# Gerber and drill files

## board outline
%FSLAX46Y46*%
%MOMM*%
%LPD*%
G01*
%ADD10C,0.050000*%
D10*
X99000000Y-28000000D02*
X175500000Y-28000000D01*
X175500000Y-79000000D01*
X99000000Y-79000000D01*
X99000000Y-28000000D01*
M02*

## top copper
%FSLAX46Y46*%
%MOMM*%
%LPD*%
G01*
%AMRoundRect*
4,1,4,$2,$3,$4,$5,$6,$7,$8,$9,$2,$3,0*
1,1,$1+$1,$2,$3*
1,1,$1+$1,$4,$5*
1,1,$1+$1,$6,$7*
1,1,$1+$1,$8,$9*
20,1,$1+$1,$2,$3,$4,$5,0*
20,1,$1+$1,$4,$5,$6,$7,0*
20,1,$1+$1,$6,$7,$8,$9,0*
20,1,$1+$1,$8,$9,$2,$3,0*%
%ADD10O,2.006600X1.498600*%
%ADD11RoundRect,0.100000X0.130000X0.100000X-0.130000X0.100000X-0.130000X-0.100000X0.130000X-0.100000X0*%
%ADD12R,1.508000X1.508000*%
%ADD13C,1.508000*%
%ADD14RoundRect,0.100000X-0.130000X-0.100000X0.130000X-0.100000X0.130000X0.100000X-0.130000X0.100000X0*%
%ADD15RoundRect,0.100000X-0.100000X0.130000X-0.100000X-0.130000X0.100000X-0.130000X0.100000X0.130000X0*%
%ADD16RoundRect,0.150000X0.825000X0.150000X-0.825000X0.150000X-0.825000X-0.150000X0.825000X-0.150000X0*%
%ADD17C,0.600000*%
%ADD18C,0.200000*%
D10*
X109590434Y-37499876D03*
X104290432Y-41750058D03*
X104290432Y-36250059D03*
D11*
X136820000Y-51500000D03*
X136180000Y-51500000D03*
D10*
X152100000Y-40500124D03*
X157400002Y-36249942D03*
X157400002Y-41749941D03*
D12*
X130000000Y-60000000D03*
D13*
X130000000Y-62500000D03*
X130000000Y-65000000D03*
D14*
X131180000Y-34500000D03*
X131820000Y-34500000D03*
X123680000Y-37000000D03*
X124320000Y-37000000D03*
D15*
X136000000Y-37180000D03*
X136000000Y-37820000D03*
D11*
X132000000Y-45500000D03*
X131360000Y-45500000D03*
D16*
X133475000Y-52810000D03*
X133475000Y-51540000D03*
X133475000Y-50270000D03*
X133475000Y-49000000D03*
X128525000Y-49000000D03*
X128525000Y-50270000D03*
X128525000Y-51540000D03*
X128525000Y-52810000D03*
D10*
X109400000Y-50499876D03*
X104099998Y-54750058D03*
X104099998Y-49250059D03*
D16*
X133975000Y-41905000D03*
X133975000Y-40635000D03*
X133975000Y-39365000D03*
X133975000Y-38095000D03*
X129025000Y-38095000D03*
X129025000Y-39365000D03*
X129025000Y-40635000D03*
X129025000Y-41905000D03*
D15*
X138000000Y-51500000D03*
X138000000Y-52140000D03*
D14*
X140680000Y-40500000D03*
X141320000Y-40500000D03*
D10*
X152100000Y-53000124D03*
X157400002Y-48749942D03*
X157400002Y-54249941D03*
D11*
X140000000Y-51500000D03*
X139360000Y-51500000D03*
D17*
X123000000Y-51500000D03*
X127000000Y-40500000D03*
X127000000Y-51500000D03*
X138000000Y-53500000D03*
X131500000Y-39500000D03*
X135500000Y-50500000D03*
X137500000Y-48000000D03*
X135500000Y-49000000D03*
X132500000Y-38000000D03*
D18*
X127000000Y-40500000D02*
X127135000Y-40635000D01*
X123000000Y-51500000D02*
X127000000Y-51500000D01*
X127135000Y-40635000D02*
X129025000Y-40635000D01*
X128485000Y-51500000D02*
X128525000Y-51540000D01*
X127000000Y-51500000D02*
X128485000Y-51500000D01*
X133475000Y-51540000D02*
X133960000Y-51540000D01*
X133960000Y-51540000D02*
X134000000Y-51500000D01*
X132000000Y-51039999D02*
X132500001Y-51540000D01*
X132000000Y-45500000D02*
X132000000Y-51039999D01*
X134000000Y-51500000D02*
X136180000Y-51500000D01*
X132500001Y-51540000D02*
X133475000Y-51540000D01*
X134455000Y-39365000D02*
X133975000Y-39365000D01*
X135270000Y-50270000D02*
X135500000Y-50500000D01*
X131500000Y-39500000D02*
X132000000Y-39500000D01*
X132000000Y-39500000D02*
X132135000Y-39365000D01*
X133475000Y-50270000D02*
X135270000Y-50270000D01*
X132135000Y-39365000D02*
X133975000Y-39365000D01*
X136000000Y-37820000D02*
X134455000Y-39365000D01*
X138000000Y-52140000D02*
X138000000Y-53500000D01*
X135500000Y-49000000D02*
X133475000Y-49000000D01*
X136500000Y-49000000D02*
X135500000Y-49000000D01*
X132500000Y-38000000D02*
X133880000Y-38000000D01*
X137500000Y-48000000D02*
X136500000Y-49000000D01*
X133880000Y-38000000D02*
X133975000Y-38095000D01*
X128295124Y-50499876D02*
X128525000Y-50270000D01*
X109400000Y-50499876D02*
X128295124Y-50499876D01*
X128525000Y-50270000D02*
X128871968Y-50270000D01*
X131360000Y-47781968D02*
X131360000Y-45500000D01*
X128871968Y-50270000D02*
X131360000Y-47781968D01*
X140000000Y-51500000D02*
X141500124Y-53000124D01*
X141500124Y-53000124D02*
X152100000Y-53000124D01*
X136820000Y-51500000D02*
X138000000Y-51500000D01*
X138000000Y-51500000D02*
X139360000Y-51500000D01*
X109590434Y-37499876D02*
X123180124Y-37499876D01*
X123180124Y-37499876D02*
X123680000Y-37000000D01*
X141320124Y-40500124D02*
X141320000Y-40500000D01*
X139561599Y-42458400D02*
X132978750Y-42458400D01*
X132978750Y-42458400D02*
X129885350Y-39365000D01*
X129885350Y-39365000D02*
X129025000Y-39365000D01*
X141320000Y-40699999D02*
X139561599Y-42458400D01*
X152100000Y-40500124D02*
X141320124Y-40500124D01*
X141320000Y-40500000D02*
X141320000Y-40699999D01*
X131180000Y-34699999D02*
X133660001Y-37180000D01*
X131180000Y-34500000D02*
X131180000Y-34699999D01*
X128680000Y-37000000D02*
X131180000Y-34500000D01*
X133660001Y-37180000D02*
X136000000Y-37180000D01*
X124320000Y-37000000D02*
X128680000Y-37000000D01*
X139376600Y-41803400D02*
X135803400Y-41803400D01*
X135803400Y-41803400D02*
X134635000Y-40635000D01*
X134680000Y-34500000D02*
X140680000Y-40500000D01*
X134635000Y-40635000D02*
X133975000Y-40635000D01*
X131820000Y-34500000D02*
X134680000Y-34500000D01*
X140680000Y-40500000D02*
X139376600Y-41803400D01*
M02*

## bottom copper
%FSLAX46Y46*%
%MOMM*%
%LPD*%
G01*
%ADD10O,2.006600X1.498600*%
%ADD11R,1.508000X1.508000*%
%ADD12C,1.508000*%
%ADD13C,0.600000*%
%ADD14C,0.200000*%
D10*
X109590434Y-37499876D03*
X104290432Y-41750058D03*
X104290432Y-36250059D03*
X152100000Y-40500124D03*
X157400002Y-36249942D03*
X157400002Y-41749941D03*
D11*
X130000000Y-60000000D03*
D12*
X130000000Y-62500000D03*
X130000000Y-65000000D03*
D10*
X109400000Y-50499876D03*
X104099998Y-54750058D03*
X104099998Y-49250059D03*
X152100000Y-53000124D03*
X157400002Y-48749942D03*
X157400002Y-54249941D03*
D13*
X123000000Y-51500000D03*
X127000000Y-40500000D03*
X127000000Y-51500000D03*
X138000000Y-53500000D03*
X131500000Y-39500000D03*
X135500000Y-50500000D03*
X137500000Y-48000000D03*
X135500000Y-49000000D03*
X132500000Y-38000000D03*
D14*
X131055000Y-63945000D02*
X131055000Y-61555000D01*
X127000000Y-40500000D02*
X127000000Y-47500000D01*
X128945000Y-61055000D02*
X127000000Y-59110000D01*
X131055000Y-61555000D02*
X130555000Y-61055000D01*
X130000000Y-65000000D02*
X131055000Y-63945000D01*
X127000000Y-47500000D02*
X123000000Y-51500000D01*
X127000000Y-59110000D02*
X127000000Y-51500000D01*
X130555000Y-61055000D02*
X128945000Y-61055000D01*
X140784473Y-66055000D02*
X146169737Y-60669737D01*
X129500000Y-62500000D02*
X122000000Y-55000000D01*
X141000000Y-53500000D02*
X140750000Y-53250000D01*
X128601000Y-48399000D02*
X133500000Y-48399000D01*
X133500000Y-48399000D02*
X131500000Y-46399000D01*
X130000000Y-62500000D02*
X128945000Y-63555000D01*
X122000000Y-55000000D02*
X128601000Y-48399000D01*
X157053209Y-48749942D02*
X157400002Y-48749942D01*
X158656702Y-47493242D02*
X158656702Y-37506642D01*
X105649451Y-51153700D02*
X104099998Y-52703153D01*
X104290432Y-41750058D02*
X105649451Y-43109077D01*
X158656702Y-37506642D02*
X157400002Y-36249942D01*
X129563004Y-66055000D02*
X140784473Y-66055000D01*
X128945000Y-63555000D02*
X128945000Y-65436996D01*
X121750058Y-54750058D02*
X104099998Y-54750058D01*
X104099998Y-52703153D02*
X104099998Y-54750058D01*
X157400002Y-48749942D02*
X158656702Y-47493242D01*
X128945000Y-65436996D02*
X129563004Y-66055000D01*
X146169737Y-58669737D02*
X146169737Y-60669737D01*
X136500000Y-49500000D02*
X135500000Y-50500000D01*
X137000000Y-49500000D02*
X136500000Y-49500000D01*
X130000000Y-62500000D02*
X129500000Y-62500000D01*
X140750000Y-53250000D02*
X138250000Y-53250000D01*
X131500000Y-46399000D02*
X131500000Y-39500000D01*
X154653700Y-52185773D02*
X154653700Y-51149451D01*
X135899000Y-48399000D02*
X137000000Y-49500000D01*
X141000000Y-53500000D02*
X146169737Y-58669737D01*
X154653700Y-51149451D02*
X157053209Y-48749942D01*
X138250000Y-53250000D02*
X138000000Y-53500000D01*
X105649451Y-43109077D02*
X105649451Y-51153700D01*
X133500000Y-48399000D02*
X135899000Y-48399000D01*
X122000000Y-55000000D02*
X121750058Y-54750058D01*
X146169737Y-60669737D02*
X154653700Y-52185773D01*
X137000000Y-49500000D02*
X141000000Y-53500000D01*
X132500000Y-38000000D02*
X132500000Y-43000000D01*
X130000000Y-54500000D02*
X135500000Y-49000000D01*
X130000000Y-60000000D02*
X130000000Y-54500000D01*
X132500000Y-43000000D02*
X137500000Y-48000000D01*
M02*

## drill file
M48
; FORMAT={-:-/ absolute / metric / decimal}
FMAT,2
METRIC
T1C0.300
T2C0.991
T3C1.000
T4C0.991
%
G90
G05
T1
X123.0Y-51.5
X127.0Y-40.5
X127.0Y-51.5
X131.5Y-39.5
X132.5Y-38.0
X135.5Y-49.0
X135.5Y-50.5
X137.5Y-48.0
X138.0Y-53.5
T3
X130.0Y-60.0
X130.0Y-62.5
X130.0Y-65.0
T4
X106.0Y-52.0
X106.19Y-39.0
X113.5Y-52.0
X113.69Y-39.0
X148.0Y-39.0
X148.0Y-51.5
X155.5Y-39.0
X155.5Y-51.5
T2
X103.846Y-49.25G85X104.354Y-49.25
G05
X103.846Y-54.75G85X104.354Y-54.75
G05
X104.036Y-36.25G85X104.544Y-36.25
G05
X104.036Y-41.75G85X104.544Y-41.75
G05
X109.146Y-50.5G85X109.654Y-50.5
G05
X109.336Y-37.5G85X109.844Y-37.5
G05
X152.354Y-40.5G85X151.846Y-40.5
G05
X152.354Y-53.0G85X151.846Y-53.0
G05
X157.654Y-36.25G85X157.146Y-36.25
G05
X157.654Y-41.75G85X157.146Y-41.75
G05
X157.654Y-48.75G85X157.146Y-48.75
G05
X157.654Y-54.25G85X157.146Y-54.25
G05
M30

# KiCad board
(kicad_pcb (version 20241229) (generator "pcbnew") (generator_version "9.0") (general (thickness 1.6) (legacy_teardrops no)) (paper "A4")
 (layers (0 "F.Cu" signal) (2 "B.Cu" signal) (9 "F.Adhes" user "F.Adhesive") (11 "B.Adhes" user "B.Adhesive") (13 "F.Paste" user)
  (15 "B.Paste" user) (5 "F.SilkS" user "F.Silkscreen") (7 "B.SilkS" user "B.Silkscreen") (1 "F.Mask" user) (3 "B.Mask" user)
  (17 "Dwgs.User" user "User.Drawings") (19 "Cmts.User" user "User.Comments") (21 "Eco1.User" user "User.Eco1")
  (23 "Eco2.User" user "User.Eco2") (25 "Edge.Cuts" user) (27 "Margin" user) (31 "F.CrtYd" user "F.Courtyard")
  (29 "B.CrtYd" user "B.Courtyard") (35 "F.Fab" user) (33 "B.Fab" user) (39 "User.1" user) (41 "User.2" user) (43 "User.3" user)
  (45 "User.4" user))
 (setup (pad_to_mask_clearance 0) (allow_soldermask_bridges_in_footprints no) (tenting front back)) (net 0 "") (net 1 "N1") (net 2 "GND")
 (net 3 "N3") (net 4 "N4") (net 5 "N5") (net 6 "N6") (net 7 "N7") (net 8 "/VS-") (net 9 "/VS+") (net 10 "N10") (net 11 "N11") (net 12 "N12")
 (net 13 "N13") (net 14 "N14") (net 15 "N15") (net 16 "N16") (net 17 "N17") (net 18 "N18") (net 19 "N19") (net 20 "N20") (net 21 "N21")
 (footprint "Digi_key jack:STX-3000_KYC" (layer "F.Cu") (at 109.590434 37.499876 -90)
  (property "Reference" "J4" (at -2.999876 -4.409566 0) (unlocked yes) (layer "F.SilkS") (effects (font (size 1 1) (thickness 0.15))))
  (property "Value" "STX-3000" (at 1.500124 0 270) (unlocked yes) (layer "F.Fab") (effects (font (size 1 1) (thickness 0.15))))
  (pad "" np_thru_hole circle (at 1.500124 -4.1 270) (size 0.9906 0.9906) (drill 0.9906) (layers "*.Cu" "*.Mask"))
  (pad "" np_thru_hole circle (at 1.500124 3.4 270) (size 0.9906 0.9906) (drill 0.9906) (layers "*.Cu" "*.Mask"))
  (pad "1" thru_hole oval (at 0 0) (size 2.0066 1.4986) (drill oval 1.4986 0.9906) (layers "*.Cu" "*.Mask") (remove_unused_layers no)
   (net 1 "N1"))
  (pad "2" thru_hole oval (at 4.250182 5.300002) (size 2.0066 1.4986) (drill oval 1.4986 0.9906) (layers "*.Cu" "*.Mask")
   (remove_unused_layers no) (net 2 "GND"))
  (pad "3" thru_hole oval (at -1.249817 5.300002) (size 2.0066 1.4986) (drill oval 1.4986 0.9906) (layers "*.Cu" "*.Mask")
   (remove_unused_layers no) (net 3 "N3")))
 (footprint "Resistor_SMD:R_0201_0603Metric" (layer "F.Cu") (at 136.5 51.5 180)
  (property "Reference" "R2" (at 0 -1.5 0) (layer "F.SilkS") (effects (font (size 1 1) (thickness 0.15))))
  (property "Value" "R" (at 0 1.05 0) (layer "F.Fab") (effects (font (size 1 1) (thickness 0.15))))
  (pad "" smd roundrect (at -0.345 0 180) (size 0.318 0.36) (layers "F.Paste") (roundrect_rratio 0.25))
  (pad "" smd roundrect (at 0.345 0 180) (size 0.318 0.36) (layers "F.Paste") (roundrect_rratio 0.25))
  (pad "1" smd roundrect (at -0.32 0 180) (size 0.46 0.4) (layers "F.Cu" "F.Mask") (roundrect_rratio 0.25) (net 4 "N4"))
  (pad "2" smd roundrect (at 0.32 0 180) (size 0.46 0.4) (layers "F.Cu" "F.Mask") (roundrect_rratio 0.25) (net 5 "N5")))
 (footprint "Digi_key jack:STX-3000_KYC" (layer "F.Cu") (at 152.1 40.500124 90)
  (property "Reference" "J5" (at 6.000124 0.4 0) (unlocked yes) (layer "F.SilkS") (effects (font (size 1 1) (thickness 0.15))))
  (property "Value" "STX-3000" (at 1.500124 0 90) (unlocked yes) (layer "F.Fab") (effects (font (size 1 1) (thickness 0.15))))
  (pad "" np_thru_hole circle (at 1.500124 -4.1 90) (size 0.9906 0.9906) (drill 0.9906) (layers "*.Cu" "*.Mask"))
  (pad "" np_thru_hole circle (at 1.500124 3.4 90) (size 0.9906 0.9906) (drill 0.9906) (layers "*.Cu" "*.Mask"))
  (pad "1" thru_hole oval (at 0 0 180) (size 2.0066 1.4986) (drill oval 1.4986 0.9906) (layers "*.Cu" "*.Mask") (remove_unused_layers no)
   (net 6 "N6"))
  (pad "2" thru_hole oval (at 4.250182 5.300002 180) (size 2.0066 1.4986) (drill oval 1.4986 0.9906) (layers "*.Cu" "*.Mask")
   (remove_unused_layers no) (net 2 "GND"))
  (pad "3" thru_hole oval (at -1.249817 5.300002 180) (size 2.0066 1.4986) (drill oval 1.4986 0.9906) (layers "*.Cu" "*.Mask")
   (remove_unused_layers no) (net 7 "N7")))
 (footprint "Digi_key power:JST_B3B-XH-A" (layer "F.Cu") (at 129.475 62.5 90)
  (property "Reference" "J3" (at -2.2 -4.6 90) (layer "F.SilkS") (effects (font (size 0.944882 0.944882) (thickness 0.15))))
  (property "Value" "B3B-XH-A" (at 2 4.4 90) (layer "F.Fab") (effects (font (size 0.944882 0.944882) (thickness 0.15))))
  (pad "1" thru_hole rect (at 2.5 0.525 90) (size 1.508 1.508) (drill 1) (layers "*.Cu" "*.Mask") (remove_unused_layers no) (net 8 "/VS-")
   (solder_mask_margin 0.102))
  (pad "2" thru_hole circle (at 0 0.525 90) (size 1.508 1.508) (drill 1) (layers "*.Cu" "*.Mask") (remove_unused_layers no) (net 2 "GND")
   (solder_mask_margin 0.102))
  (pad "3" thru_hole circle (at -2.5 0.525 90) (size 1.508 1.508) (drill 1) (layers "*.Cu" "*.Mask") (remove_unused_layers no)
   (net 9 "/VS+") (solder_mask_margin 0.102)))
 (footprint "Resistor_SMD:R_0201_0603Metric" (layer "F.Cu") (at 131.5 34.5)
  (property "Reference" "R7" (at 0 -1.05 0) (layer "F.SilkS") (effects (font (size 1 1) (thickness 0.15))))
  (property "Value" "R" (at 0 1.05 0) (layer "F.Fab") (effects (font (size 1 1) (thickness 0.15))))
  (pad "" smd roundrect (at -0.345 0) (size 0.318 0.36) (layers "F.Paste") (roundrect_rratio 0.25))
  (pad "" smd roundrect (at 0.345 0) (size 0.318 0.36) (layers "F.Paste") (roundrect_rratio 0.25))
  (pad "1" smd roundrect (at -0.32 0) (size 0.46 0.4) (layers "F.Cu" "F.Mask") (roundrect_rratio 0.25) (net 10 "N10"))
  (pad "2" smd roundrect (at 0.32 0) (size 0.46 0.4) (layers "F.Cu" "F.Mask") (roundrect_rratio 0.25) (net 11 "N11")))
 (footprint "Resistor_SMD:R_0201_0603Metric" (layer "F.Cu") (at 124 37)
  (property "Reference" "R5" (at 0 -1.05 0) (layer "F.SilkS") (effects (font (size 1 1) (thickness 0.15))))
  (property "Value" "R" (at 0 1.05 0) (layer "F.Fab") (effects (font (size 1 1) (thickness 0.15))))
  (pad "" smd roundrect (at -0.345 0) (size 0.318 0.36) (layers "F.Paste") (roundrect_rratio 0.25))
  (pad "" smd roundrect (at 0.345 0) (size 0.318 0.36) (layers "F.Paste") (roundrect_rratio 0.25))
  (pad "1" smd roundrect (at -0.32 0) (size 0.46 0.4) (layers "F.Cu" "F.Mask") (roundrect_rratio 0.25) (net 1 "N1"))
  (pad "2" smd roundrect (at 0.32 0) (size 0.46 0.4) (layers "F.Cu" "F.Mask") (roundrect_rratio 0.25) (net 10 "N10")))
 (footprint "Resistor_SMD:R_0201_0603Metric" (layer "F.Cu") (at 136 37.5 -90)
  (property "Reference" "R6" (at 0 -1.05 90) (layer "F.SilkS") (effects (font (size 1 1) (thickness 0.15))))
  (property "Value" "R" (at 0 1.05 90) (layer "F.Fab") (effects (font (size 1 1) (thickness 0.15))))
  (pad "" smd roundrect (at -0.345 0 270) (size 0.318 0.36) (layers "F.Paste") (roundrect_rratio 0.25))
  (pad "" smd roundrect (at 0.345 0 270) (size 0.318 0.36) (layers "F.Paste") (roundrect_rratio 0.25))
  (pad "1" smd roundrect (at -0.32 0 270) (size 0.46 0.4) (layers "F.Cu" "F.Mask") (roundrect_rratio 0.25) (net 10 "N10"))
  (pad "2" smd roundrect (at 0.32 0 270) (size 0.46 0.4) (layers "F.Cu" "F.Mask") (roundrect_rratio 0.25) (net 2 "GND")))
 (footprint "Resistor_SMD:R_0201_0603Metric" (layer "F.Cu") (at 131.68 45.5 180)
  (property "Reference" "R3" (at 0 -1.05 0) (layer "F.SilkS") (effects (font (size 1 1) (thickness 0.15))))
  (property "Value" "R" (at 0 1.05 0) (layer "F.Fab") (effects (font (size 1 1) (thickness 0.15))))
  (pad "" smd roundrect (at -0.345 0 180) (size 0.318 0.36) (layers "F.Paste") (roundrect_rratio 0.25))
  (pad "" smd roundrect (at 0.345 0 180) (size 0.318 0.36) (layers "F.Paste") (roundrect_rratio 0.25))
  (pad "1" smd roundrect (at -0.32 0 180) (size 0.46 0.4) (layers "F.Cu" "F.Mask") (roundrect_rratio 0.25) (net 5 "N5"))
  (pad "2" smd roundrect (at 0.32 0 180) (size 0.46 0.4) (layers "F.Cu" "F.Mask") (roundrect_rratio 0.25) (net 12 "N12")))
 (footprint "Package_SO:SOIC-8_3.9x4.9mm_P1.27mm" (layer "F.Cu") (at 131 50.905 180)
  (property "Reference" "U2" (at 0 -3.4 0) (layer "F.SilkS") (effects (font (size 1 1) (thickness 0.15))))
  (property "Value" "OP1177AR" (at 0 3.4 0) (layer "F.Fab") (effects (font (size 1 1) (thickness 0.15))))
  (pad "1" smd roundrect (at -2.475 -1.905 180) (size 1.95 0.6) (layers "F.Cu" "F.Mask" "F.Paste") (roundrect_rratio 0.25) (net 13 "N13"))
  (pad "2" smd roundrect (at -2.475 -0.635 180) (size 1.95 0.6) (layers "F.Cu" "F.Mask" "F.Paste") (roundrect_rratio 0.25) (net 5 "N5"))
  (pad "3" smd roundrect (at -2.475 0.635 180) (size 1.95 0.6) (layers "F.Cu" "F.Mask" "F.Paste") (roundrect_rratio 0.25) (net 2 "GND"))
  (pad "4" smd roundrect (at -2.475 1.905 180) (size 1.95 0.6) (layers "F.Cu" "F.Mask" "F.Paste") (roundrect_rratio 0.25) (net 8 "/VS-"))
  (pad "5" smd roundrect (at 2.475 1.905 180) (size 1.95 0.6) (layers "F.Cu" "F.Mask" "F.Paste") (roundrect_rratio 0.25) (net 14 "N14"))
  (pad "6" smd roundrect (at 2.475 0.635 180) (size 1.95 0.6) (layers "F.Cu" "F.Mask" "F.Paste") (roundrect_rratio 0.25) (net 12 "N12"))
  (pad "7" smd roundrect (at 2.475 -0.635 180) (size 1.95 0.6) (layers "F.Cu" "F.Mask" "F.Paste") (roundrect_rratio 0.25) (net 9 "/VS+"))
  (pad "8" smd roundrect (at 2.475 -1.905 180) (size 1.95 0.6) (layers "F.Cu" "F.Mask" "F.Paste") (roundrect_rratio 0.25) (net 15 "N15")))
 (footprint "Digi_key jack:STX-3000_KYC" (layer "F.Cu") (at 109.4 50.499876 -90)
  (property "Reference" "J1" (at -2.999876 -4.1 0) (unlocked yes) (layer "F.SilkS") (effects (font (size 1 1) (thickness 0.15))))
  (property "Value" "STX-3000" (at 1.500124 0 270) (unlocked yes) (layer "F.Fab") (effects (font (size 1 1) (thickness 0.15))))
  (pad "" np_thru_hole circle (at 1.500124 -4.1 270) (size 0.9906 0.9906) (drill 0.9906) (layers "*.Cu" "*.Mask"))
  (pad "" np_thru_hole circle (at 1.500124 3.4 270) (size 0.9906 0.9906) (drill 0.9906) (layers "*.Cu" "*.Mask"))
  (pad "1" thru_hole oval (at 0 0) (size 2.0066 1.4986) (drill oval 1.4986 0.9906) (layers "*.Cu" "*.Mask") (remove_unused_layers no)
   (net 12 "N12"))
  (pad "2" thru_hole oval (at 4.250182 5.300002) (size 2.0066 1.4986) (drill oval 1.4986 0.9906) (layers "*.Cu" "*.Mask")
   (remove_unused_layers no) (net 2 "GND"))
  (pad "3" thru_hole oval (at -1.249817 5.300002) (size 2.0066 1.4986) (drill oval 1.4986 0.9906) (layers "*.Cu" "*.Mask")
   (remove_unused_layers no) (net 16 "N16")))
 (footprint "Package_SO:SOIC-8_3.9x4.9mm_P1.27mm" (layer "F.Cu") (at 131.5 40 180)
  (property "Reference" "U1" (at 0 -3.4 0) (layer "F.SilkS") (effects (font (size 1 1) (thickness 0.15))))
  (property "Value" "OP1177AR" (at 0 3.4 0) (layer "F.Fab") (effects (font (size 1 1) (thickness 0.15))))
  (pad "1" smd roundrect (at -2.475 -1.905 180) (size 1.95 0.6) (layers "F.Cu" "F.Mask" "F.Paste") (roundrect_rratio 0.25) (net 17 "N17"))
  (pad "2" smd roundrect (at -2.475 -0.635 180) (size 1.95 0.6) (layers "F.Cu" "F.Mask" "F.Paste") (roundrect_rratio 0.25) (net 11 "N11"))
  (pad "3" smd roundrect (at -2.475 0.635 180) (size 1.95 0.6) (layers "F.Cu" "F.Mask" "F.Paste") (roundrect_rratio 0.25) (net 2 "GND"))
  (pad "4" smd roundrect (at -2.475 1.905 180) (size 1.95 0.6) (layers "F.Cu" "F.Mask" "F.Paste") (roundrect_rratio 0.25) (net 8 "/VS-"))
  (pad "5" smd roundrect (at 2.475 1.905 180) (size 1.95 0.6) (layers "F.Cu" "F.Mask" "F.Paste") (roundrect_rratio 0.25) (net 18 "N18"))
  (pad "6" smd roundrect (at 2.475 0.635 180) (size 1.95 0.6) (layers "F.Cu" "F.Mask" "F.Paste") (roundrect_rratio 0.25) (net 6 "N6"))
  (pad "7" smd roundrect (at 2.475 -0.635 180) (size 1.95 0.6) (layers "F.Cu" "F.Mask" "F.Paste") (roundrect_rratio 0.25) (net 9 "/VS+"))
  (pad "8" smd roundrect (at 2.475 -1.905 180) (size 1.95 0.6) (layers "F.Cu" "F.Mask" "F.Paste") (roundrect_rratio 0.25) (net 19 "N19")))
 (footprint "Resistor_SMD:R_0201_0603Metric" (layer "F.Cu") (at 138 51.82 -90)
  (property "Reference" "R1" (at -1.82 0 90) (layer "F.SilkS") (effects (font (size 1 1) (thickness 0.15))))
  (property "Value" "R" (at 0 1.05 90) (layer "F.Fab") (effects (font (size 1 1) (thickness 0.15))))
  (pad "" smd roundrect (at -0.345 0 270) (size 0.318 0.36) (layers "F.Paste") (roundrect_rratio 0.25))
  (pad "" smd roundrect (at 0.345 0 270) (size 0.318 0.36) (layers "F.Paste") (roundrect_rratio 0.25))
  (pad "1" smd roundrect (at -0.32 0 270) (size 0.46 0.4) (layers "F.Cu" "F.Mask") (roundrect_rratio 0.25) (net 4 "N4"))
  (pad "2" smd roundrect (at 0.32 0 270) (size 0.46 0.4) (layers "F.Cu" "F.Mask") (roundrect_rratio 0.25) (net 2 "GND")))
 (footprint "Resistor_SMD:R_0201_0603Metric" (layer "F.Cu") (at 141 40.5)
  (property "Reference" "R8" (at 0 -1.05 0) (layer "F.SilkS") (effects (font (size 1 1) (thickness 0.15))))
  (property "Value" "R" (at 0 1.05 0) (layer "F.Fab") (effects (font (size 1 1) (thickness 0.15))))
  (pad "" smd roundrect (at -0.345 0) (size 0.318 0.36) (layers "F.Paste") (roundrect_rratio 0.25))
  (pad "" smd roundrect (at 0.345 0) (size 0.318 0.36) (layers "F.Paste") (roundrect_rratio 0.25))
  (pad "1" smd roundrect (at -0.32 0) (size 0.46 0.4) (layers "F.Cu" "F.Mask") (roundrect_rratio 0.25) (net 11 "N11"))
  (pad "2" smd roundrect (at 0.32 0) (size 0.46 0.4) (layers "F.Cu" "F.Mask") (roundrect_rratio 0.25) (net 6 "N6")))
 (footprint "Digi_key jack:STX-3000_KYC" (layer "F.Cu") (at 152.1 53.000124 90)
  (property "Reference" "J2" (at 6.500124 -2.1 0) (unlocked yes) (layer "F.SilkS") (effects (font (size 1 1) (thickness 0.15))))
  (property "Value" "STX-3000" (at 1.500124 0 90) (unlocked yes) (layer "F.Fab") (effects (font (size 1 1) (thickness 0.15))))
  (pad "" np_thru_hole circle (at 1.500124 -4.1 90) (size 0.9906 0.9906) (drill 0.9906) (layers "*.Cu" "*.Mask"))
  (pad "" np_thru_hole circle (at 1.500124 3.4 90) (size 0.9906 0.9906) (drill 0.9906) (layers "*.Cu" "*.Mask"))
  (pad "1" thru_hole oval (at 0 0 180) (size 2.0066 1.4986) (drill oval 1.4986 0.9906) (layers "*.Cu" "*.Mask") (remove_unused_layers no)
   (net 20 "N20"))
  (pad "2" thru_hole oval (at 4.250182 5.300002 180) (size 2.0066 1.4986) (drill oval 1.4986 0.9906) (layers "*.Cu" "*.Mask")
   (remove_unused_layers no) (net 2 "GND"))
  (pad "3" thru_hole oval (at -1.249817 5.300002 180) (size 2.0066 1.4986) (drill oval 1.4986 0.9906) (layers "*.Cu" "*.Mask")
   (remove_unused_layers no) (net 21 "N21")))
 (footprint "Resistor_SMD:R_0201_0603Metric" (layer "F.Cu") (at 139.68 51.5 180)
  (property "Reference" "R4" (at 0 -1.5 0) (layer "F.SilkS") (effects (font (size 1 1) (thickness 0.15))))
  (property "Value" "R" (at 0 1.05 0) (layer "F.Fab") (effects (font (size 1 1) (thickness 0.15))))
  (pad "" smd roundrect (at -0.345 0 180) (size 0.318 0.36) (layers "F.Paste") (roundrect_rratio 0.25))
  (pad "" smd roundrect (at 0.345 0 180) (size 0.318 0.36) (layers "F.Paste") (roundrect_rratio 0.25))
  (pad "1" smd roundrect (at -0.32 0 180) (size 0.46 0.4) (layers "F.Cu" "F.Mask") (roundrect_rratio 0.25) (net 20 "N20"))
  (pad "2" smd roundrect (at 0.32 0 180) (size 0.46 0.4) (layers "F.Cu" "F.Mask") (roundrect_rratio 0.25) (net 4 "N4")))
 (gr_rect (start 99 28) (end 175.5 79) (stroke (width 0.05) (type default)) (fill no) (layer "Edge.Cuts"))
 (segment (start 127 40.5) (end 127.135 40.635) (width 0.2) (layer "F.Cu") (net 9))
 (segment (start 123 51.5) (end 127 51.5) (width 0.2) (layer "F.Cu") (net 9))
 (segment (start 127.135 40.635) (end 129.025 40.635) (width 0.2) (layer "F.Cu") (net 9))
 (segment (start 128.485 51.5) (end 128.525 51.54) (width 0.2) (layer "F.Cu") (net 9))
 (segment (start 127 51.5) (end 128.485 51.5) (width 0.2) (layer "F.Cu") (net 9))
 (via (at 123 51.5) (size 0.6) (drill 0.3) (layers "F.Cu" "B.Cu") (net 9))
 (via (at 127 40.5) (size 0.6) (drill 0.3) (layers "F.Cu" "B.Cu") (free yes) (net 9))
 (via (at 127 51.5) (size 0.6) (drill 0.3) (layers "F.Cu" "B.Cu") (free yes) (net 9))
 (segment (start 131.055 63.945) (end 131.055 61.555) (width 0.2) (layer "B.Cu") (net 9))
 (segment (start 127 40.5) (end 127 47.5) (width 0.2) (layer "B.Cu") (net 9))
 (segment (start 128.945 61.055) (end 127 59.11) (width 0.2) (layer "B.Cu") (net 9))
 (segment (start 131.055 61.555) (end 130.555 61.055) (width 0.2) (layer "B.Cu") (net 9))
 (segment (start 130 65) (end 131.055 63.945) (width 0.2) (layer "B.Cu") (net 9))
 (segment (start 127 47.5) (end 123 51.5) (width 0.2) (layer "B.Cu") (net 9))
 (segment (start 127 59.11) (end 127 51.5) (width 0.2) (layer "B.Cu") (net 9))
 (segment (start 130.555 61.055) (end 128.945 61.055) (width 0.2) (layer "B.Cu") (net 9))
 (segment (start 133.475 51.54) (end 133.96 51.54) (width 0.2) (layer "F.Cu") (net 5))
 (segment (start 133.96 51.54) (end 134 51.5) (width 0.2) (layer "F.Cu") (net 5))
 (segment (start 132 51.039999) (end 132.500001 51.54) (width 0.2) (layer "F.Cu") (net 5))
 (segment (start 132 45.5) (end 132 51.039999) (width 0.2) (layer "F.Cu") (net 5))
 (segment (start 134 51.5) (end 136.18 51.5) (width 0.2) (layer "F.Cu") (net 5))
 (segment (start 132.500001 51.54) (end 133.475 51.54) (width 0.2) (layer "F.Cu") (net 5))
 (segment (start 134.455 39.365) (end 133.975 39.365) (width 0.2) (layer "F.Cu") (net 2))
 (segment (start 135.27 50.27) (end 135.5 50.5) (width 0.2) (layer "F.Cu") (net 2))
 (segment (start 131.5 39.5) (end 132 39.5) (width 0.2) (layer "F.Cu") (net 2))
 (segment (start 132 39.5) (end 132.135 39.365) (width 0.2) (layer "F.Cu") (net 2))
 (segment (start 133.475 50.27) (end 135.27 50.27) (width 0.2) (layer "F.Cu") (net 2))
 (segment (start 132.135 39.365) (end 133.975 39.365) (width 0.2) (layer "F.Cu") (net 2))
 (segment (start 136 37.82) (end 134.455 39.365) (width 0.2) (layer "F.Cu") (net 2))
 (segment (start 138 52.14) (end 138 53.5) (width 0.2) (layer "F.Cu") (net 2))
 (via (at 138 53.5) (size 0.6) (drill 0.3) (layers "F.Cu" "B.Cu") (free yes) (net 2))
 (via (at 131.5 39.5) (size 0.6) (drill 0.3) (layers "F.Cu" "B.Cu") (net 2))
 (via (at 135.5 50.5) (size 0.6) (drill 0.3) (layers "F.Cu" "B.Cu") (free yes) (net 2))
 (segment (start 140.784473 66.055) (end 146.169737 60.669737) (width 0.2) (layer "B.Cu") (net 2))
 (segment (start 129.5 62.5) (end 122 55) (width 0.2) (layer "B.Cu") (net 2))
 (segment (start 141 53.5) (end 140.75 53.25) (width 0.2) (layer "B.Cu") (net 2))
 (segment (start 128.601 48.399) (end 133.5 48.399) (width 0.2) (layer "B.Cu") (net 2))
 (segment (start 133.5 48.399) (end 131.5 46.399) (width 0.2) (layer "B.Cu") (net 2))
 (segment (start 130 62.5) (end 128.945 63.555) (width 0.2) (layer "B.Cu") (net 2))
 (segment (start 122 55) (end 128.601 48.399) (width 0.2) (layer "B.Cu") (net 2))
 (segment (start 157.053209 48.749942) (end 157.400002 48.749942) (width 0.2) (layer "B.Cu") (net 2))
 (segment (start 158.656702 47.493242) (end 158.656702 37.506642) (width 0.2) (layer "B.Cu") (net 2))
 (segment (start 105.649451 51.1537) (end 104.099998 52.703153) (width 0.2) (layer "B.Cu") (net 2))
 (segment (start 104.290432 41.750058) (end 105.649451 43.109077) (width 0.2) (layer "B.Cu") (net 2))
 (segment (start 158.656702 37.506642) (end 157.400002 36.249942) (width 0.2) (layer "B.Cu") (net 2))
 (segment (start 129.563004 66.055) (end 140.784473 66.055) (width 0.2) (layer "B.Cu") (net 2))
 (segment (start 128.945 63.555) (end 128.945 65.436996) (width 0.2) (layer "B.Cu") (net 2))
 (segment (start 121.750058 54.750058) (end 104.099998 54.750058) (width 0.2) (layer "B.Cu") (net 2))
 (segment (start 104.099998 52.703153) (end 104.099998 54.750058) (width 0.2) (layer "B.Cu") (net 2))
 (segment (start 157.400002 48.749942) (end 158.656702 47.493242) (width 0.2) (layer "B.Cu") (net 2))
 (segment (start 128.945 65.436996) (end 129.563004 66.055) (width 0.2) (layer "B.Cu") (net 2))
 (segment (start 146.169737 58.669737) (end 146.169737 60.669737) (width 0.2) (layer "B.Cu") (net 2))
 (segment (start 136.5 49.5) (end 135.5 50.5) (width 0.2) (layer "B.Cu") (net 2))
 (segment (start 137 49.5) (end 136.5 49.5) (width 0.2) (layer "B.Cu") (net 2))
 (segment (start 130 62.5) (end 129.5 62.5) (width 0.2) (layer "B.Cu") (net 2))
 (segment (start 140.75 53.25) (end 138.25 53.25) (width 0.2) (layer "B.Cu") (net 2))
 (segment (start 131.5 46.399) (end 131.5 39.5) (width 0.2) (layer "B.Cu") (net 2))
 (segment (start 154.6537 52.185773) (end 154.6537 51.149451) (width 0.2) (layer "B.Cu") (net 2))
 (segment (start 135.899 48.399) (end 137 49.5) (width 0.2) (layer "B.Cu") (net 2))
 (segment (start 141 53.5) (end 146.169737 58.669737) (width 0.2) (layer "B.Cu") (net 2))
 (segment (start 154.6537 51.149451) (end 157.053209 48.749942) (width 0.2) (layer "B.Cu") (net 2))
 (segment (start 138.25 53.25) (end 138 53.5) (width 0.2) (layer "B.Cu") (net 2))
 (segment (start 105.649451 43.109077) (end 105.649451 51.1537) (width 0.2) (layer "B.Cu") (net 2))
 (segment (start 133.5 48.399) (end 135.899 48.399) (width 0.2) (layer "B.Cu") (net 2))
 (segment (start 122 55) (end 121.750058 54.750058) (width 0.2) (layer "B.Cu") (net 2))
 (segment (start 146.169737 60.669737) (end 154.6537 52.185773) (width 0.2) (layer "B.Cu") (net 2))
 (segment (start 137 49.5) (end 141 53.5) (width 0.2) (layer "B.Cu") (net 2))
 (segment (start 135.5 49) (end 133.475 49) (width 0.2) (layer "F.Cu") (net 8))
 (segment (start 136.5 49) (end 135.5 49) (width 0.2) (layer "F.Cu") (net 8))
 (segment (start 132.5 38) (end 133.88 38) (width 0.2) (layer "F.Cu") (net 8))
 (segment (start 137.5 48) (end 136.5 49) (width 0.2) (layer "F.Cu") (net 8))
 (segment (start 133.88 38) (end 133.975 38.095) (width 0.2) (layer "F.Cu") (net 8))
 (via (at 137.5 48) (size 0.6) (drill 0.3) (layers "F.Cu" "B.Cu") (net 8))
 (via (at 135.5 49) (size 0.6) (drill 0.3) (layers "F.Cu" "B.Cu") (free yes) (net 8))
 (via (at 132.5 38) (size 0.6) (drill 0.3) (layers "F.Cu" "B.Cu") (free yes) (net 8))
 (segment (start 132.5 38) (end 132.5 43) (width 0.2) (layer "B.Cu") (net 8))
 (segment (start 130 54.5) (end 135.5 49) (width 0.2) (layer "B.Cu") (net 8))
 (segment (start 130 60) (end 130 54.5) (width 0.2) (layer "B.Cu") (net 8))
 (segment (start 132.5 43) (end 137.5 48) (width 0.2) (layer "B.Cu") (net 8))
 (segment (start 128.295124 50.499876) (end 128.525 50.27) (width 0.2) (layer "F.Cu") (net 12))
 (segment (start 109.4 50.499876) (end 128.295124 50.499876) (width 0.2) (layer "F.Cu") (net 12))
 (segment (start 128.525 50.27) (end 128.871968 50.27) (width 0.2) (layer "F.Cu") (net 12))
 (segment (start 131.36 47.781968) (end 131.36 45.5) (width 0.2) (layer "F.Cu") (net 12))
 (segment (start 128.871968 50.27) (end 131.36 47.781968) (width 0.2) (layer "F.Cu") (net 12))
 (segment (start 140 51.5) (end 141.500124 53.000124) (width 0.2) (layer "F.Cu") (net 20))
 (segment (start 141.500124 53.000124) (end 152.1 53.000124) (width 0.2) (layer "F.Cu") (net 20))
 (segment (start 136.82 51.5) (end 138 51.5) (width 0.2) (layer "F.Cu") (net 4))
 (segment (start 138 51.5) (end 139.36 51.5) (width 0.2) (layer "F.Cu") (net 4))
 (segment (start 109.590434 37.499876) (end 123.180124 37.499876) (width 0.2) (layer "F.Cu") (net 1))
 (segment (start 123.180124 37.499876) (end 123.68 37) (width 0.2) (layer "F.Cu") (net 1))
 (segment (start 141.320124 40.500124) (end 141.32 40.5) (width 0.2) (layer "F.Cu") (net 6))
 (segment (start 139.561599 42.4584) (end 132.97875 42.4584) (width 0.2) (layer "F.Cu") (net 6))
 (segment (start 132.97875 42.4584) (end 129.88535 39.365) (width 0.2) (layer "F.Cu") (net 6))
 (segment (start 129.88535 39.365) (end 129.025 39.365) (width 0.2) (layer "F.Cu") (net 6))
 (segment (start 141.32 40.699999) (end 139.561599 42.4584) (width 0.2) (layer "F.Cu") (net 6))
 (segment (start 152.1 40.500124) (end 141.320124 40.500124) (width 0.2) (layer "F.Cu") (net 6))
 (segment (start 141.32 40.5) (end 141.32 40.699999) (width 0.2) (layer "F.Cu") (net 6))
 (segment (start 131.18 34.699999) (end 133.660001 37.18) (width 0.2) (layer "F.Cu") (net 10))
 (segment (start 131.18 34.5) (end 131.18 34.699999) (width 0.2) (layer "F.Cu") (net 10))
 (segment (start 128.68 37) (end 131.18 34.5) (width 0.2) (layer "F.Cu") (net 10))
 (segment (start 133.660001 37.18) (end 136 37.18) (width 0.2) (layer "F.Cu") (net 10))
 (segment (start 124.32 37) (end 128.68 37) (width 0.2) (layer "F.Cu") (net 10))
 (segment (start 139.3766 41.8034) (end 135.8034 41.8034) (width 0.2) (layer "F.Cu") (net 11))
 (segment (start 135.8034 41.8034) (end 134.635 40.635) (width 0.2) (layer "F.Cu") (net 11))
 (segment (start 134.68 34.5) (end 140.68 40.5) (width 0.2) (layer "F.Cu") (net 11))
 (segment (start 134.635 40.635) (end 133.975 40.635) (width 0.2) (layer "F.Cu") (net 11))
 (segment (start 131.82 34.5) (end 134.68 34.5) (width 0.2) (layer "F.Cu") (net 11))
 (segment (start 140.68 40.5) (end 139.3766 41.8034) (width 0.2) (layer "F.Cu") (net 11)))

